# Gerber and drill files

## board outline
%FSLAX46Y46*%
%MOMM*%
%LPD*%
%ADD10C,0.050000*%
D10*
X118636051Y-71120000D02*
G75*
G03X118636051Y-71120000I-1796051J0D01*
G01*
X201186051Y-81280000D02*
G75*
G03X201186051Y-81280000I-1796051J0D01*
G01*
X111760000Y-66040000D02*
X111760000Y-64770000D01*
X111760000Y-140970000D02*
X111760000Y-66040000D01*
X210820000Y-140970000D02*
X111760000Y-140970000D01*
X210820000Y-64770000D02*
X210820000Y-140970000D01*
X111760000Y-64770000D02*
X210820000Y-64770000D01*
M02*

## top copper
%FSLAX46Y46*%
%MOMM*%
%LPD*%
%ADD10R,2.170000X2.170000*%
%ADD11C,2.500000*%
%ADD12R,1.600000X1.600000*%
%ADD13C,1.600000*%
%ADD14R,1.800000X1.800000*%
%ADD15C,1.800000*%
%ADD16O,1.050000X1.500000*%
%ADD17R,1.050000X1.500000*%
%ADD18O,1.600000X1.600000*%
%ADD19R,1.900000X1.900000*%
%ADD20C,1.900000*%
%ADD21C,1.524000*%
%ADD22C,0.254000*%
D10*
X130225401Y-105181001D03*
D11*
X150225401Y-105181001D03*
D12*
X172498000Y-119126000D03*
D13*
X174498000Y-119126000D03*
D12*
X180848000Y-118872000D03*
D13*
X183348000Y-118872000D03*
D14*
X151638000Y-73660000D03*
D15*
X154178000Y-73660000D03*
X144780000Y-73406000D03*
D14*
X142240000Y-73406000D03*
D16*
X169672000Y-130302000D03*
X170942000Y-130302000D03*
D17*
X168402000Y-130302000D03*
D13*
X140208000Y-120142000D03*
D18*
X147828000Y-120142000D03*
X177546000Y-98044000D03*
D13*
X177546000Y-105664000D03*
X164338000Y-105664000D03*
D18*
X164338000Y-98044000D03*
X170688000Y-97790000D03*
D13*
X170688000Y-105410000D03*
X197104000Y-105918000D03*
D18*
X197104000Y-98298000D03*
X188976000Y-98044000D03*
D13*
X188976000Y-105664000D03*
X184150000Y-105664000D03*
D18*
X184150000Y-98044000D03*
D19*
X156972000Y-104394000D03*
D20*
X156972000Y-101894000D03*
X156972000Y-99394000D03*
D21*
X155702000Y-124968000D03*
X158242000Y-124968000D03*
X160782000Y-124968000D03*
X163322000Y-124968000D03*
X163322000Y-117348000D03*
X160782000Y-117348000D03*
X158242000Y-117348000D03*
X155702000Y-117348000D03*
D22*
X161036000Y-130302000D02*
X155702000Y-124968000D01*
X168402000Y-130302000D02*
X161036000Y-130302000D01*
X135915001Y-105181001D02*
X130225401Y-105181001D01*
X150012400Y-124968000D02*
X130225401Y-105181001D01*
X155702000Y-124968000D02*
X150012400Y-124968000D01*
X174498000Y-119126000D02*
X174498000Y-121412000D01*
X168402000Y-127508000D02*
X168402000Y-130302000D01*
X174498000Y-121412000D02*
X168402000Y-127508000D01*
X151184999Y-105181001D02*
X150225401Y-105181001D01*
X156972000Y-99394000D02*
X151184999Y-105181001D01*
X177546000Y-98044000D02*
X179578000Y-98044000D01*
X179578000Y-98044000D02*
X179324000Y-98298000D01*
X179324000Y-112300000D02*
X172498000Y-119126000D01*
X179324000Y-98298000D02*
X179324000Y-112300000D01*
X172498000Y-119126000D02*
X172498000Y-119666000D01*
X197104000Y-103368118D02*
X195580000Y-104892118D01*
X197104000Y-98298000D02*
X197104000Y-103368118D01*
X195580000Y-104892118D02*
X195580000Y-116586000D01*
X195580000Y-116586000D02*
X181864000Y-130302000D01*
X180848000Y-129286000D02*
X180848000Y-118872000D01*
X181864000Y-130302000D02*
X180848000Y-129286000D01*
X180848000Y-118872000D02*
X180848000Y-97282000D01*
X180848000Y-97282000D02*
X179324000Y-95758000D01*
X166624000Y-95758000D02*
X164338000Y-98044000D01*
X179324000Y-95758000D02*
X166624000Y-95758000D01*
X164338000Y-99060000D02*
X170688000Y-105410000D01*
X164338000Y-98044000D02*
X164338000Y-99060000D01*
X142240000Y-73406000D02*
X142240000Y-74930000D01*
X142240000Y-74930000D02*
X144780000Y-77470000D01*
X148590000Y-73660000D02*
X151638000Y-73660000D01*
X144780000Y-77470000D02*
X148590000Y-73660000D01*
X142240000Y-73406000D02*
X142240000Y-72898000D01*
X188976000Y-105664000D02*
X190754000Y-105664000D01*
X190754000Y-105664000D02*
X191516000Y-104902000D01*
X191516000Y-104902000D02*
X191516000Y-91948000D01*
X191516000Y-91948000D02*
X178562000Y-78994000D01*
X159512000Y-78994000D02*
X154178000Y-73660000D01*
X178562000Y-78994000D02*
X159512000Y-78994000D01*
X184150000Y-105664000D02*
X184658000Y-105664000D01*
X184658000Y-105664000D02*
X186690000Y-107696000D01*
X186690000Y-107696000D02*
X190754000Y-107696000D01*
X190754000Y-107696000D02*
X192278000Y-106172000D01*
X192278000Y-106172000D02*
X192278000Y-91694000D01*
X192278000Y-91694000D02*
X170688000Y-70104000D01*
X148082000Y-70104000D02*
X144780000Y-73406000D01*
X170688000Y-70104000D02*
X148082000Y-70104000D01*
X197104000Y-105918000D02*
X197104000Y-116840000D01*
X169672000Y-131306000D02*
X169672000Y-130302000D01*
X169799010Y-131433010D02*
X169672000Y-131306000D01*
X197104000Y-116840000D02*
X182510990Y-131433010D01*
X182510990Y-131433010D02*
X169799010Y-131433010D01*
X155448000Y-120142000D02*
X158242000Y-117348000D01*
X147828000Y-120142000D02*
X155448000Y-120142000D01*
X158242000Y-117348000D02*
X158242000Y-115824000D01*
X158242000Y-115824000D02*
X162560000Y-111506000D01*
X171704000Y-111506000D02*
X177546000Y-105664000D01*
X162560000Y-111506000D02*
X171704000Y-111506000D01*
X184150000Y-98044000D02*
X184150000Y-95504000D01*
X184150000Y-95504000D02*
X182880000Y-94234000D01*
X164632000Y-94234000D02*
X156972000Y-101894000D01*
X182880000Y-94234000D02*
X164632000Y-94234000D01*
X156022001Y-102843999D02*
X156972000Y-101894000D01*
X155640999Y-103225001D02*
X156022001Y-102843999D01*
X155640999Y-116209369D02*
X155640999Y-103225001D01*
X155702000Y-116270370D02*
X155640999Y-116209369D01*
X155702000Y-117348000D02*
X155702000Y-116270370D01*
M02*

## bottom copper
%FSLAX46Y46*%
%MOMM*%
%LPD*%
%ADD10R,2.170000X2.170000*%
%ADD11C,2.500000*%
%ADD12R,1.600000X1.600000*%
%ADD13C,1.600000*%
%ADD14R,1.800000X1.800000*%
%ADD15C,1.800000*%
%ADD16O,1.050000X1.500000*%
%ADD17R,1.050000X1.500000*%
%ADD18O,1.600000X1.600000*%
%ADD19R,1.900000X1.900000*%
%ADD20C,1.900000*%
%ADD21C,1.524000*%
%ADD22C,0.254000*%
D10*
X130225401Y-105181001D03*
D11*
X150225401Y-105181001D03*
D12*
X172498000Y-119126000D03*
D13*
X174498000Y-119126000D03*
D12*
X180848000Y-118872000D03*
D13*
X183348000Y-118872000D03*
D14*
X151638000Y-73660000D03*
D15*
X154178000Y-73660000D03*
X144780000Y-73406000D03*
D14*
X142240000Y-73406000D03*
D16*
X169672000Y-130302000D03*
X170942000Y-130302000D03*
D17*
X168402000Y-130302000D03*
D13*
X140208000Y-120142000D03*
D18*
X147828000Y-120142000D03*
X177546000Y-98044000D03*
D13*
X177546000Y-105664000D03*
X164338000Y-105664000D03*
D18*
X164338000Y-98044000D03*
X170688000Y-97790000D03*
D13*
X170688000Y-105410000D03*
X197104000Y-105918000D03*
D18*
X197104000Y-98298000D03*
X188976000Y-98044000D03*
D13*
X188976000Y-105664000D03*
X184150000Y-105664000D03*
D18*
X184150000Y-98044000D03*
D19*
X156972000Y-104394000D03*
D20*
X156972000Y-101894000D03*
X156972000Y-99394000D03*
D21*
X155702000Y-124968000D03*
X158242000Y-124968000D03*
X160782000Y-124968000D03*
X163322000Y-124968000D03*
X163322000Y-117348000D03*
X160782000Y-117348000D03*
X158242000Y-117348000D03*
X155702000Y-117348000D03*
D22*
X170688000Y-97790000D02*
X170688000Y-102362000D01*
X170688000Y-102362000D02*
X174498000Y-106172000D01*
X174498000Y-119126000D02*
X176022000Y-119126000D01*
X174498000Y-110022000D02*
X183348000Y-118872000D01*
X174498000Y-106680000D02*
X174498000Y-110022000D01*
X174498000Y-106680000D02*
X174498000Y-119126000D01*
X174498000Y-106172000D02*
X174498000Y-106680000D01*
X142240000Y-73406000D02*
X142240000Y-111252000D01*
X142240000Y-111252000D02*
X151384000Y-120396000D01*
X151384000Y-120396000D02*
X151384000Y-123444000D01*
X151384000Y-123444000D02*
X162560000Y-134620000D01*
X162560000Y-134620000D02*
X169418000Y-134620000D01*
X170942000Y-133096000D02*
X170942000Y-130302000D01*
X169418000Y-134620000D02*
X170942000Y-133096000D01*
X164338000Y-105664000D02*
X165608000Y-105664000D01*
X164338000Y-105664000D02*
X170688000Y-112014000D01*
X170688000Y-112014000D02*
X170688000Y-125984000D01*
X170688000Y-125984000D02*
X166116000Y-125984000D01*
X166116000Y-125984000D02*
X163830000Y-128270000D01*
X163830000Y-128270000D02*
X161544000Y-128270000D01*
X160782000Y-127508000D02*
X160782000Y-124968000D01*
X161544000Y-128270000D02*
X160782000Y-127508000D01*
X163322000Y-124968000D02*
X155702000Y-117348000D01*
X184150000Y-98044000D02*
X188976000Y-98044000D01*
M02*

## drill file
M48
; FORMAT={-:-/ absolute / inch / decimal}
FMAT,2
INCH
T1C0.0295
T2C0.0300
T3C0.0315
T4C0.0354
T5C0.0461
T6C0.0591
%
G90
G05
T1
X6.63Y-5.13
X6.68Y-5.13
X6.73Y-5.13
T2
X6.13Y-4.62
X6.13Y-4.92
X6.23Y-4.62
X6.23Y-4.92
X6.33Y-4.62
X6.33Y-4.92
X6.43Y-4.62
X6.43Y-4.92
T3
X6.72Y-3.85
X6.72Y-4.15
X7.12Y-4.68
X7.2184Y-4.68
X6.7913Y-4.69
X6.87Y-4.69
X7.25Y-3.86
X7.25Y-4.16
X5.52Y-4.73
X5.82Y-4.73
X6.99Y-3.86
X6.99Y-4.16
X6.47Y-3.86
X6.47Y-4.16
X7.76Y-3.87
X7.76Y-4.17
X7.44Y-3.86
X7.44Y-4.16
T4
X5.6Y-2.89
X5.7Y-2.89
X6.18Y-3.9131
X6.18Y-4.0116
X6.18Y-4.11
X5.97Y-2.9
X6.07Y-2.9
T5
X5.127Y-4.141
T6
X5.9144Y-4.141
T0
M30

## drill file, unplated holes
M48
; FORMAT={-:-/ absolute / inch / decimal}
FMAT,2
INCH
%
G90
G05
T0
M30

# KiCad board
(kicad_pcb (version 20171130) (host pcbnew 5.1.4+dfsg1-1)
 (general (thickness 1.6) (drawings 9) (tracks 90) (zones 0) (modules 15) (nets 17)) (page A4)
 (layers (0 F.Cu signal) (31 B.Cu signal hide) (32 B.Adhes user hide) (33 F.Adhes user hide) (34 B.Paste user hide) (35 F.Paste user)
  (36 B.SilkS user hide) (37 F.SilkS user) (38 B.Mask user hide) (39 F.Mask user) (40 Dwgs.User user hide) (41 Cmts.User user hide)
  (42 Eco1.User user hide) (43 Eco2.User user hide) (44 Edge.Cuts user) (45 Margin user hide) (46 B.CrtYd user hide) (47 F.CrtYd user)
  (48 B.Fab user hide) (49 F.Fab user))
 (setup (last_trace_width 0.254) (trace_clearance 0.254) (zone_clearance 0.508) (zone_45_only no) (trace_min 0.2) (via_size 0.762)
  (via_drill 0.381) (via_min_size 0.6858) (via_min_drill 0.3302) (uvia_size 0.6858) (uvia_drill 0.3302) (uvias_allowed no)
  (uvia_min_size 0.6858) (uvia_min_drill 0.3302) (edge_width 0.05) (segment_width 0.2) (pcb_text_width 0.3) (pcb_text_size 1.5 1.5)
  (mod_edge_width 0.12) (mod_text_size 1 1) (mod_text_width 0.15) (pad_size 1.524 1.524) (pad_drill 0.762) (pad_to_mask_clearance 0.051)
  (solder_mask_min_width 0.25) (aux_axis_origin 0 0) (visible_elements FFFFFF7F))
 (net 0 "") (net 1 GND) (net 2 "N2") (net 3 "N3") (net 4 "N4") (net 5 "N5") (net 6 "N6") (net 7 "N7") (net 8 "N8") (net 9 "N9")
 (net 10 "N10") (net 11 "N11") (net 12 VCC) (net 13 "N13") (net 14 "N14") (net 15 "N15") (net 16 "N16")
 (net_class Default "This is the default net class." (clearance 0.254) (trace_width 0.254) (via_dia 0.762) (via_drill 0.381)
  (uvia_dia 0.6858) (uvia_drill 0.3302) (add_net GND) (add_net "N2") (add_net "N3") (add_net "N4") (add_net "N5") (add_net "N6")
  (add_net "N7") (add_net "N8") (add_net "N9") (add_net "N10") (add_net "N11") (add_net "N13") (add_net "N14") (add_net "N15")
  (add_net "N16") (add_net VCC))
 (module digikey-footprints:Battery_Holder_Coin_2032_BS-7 (layer F.Cu) (at 130.225401 105.181001)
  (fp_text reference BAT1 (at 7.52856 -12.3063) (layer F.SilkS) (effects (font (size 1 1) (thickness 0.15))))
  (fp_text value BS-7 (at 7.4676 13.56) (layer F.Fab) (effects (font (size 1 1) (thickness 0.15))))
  (pad Neg thru_hole rect (at 0 0) (size 2.17 2.17) (drill 1.17) (layers *.Cu *.Mask) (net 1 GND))
  (pad Pos thru_hole circle (at 20 0) (size 2.5 2.5) (drill 1.5) (layers *.Cu *.Mask) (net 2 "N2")))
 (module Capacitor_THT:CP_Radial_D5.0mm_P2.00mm (layer F.Cu) (at 172.498 119.126)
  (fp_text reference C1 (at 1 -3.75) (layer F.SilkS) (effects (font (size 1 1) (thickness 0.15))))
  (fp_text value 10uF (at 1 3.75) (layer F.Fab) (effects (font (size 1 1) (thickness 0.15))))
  (pad 1 thru_hole rect (at 0 0) (size 1.6 1.6) (drill 0.8) (layers *.Cu *.Mask) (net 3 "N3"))
  (pad 2 thru_hole circle (at 2 0) (size 1.6 1.6) (drill 0.8) (layers *.Cu *.Mask) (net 1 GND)))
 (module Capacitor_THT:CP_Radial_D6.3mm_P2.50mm (layer F.Cu) (at 180.848 118.872)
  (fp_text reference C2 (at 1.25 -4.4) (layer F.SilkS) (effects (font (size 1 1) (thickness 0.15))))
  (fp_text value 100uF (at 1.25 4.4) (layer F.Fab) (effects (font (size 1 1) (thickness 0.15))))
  (pad 1 thru_hole rect (at 0 0) (size 1.6 1.6) (drill 0.8) (layers *.Cu *.Mask) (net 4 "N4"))
  (pad 2 thru_hole circle (at 2.5 0) (size 1.6 1.6) (drill 0.8) (layers *.Cu *.Mask) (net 1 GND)))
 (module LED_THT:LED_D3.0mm (layer F.Cu) (at 151.638 73.66)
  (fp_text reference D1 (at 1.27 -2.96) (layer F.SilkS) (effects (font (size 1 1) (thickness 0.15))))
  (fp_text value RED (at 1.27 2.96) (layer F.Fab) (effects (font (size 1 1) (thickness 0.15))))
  (pad 1 thru_hole rect (at 0 0) (size 1.8 1.8) (drill 0.9) (layers *.Cu *.Mask) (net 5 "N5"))
  (pad 2 thru_hole circle (at 2.54 0) (size 1.8 1.8) (drill 0.9) (layers *.Cu *.Mask) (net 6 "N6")))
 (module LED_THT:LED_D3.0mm (layer F.Cu) (at 142.24 73.406)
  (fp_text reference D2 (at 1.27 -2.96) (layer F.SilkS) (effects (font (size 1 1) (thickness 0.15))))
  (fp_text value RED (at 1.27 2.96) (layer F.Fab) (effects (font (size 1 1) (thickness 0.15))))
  (pad 2 thru_hole circle (at 2.54 0) (size 1.8 1.8) (drill 0.9) (layers *.Cu *.Mask) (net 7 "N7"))
  (pad 1 thru_hole rect (at 0 0) (size 1.8 1.8) (drill 0.9) (layers *.Cu *.Mask) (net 5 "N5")))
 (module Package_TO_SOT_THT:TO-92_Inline (layer F.Cu) (at 168.402 130.302)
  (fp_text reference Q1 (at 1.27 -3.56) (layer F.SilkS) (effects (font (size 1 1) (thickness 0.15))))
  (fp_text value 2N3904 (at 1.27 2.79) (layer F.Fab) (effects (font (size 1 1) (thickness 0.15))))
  (pad 2 thru_hole oval (at 1.27 0) (size 1.05 1.5) (drill 0.75) (layers *.Cu *.Mask) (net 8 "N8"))
  (pad 3 thru_hole oval (at 2.54 0) (size 1.05 1.5) (drill 0.75) (layers *.Cu *.Mask) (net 5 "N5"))
  (pad 1 thru_hole rect (at 0 0) (size 1.05 1.5) (drill 0.75) (layers *.Cu *.Mask) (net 1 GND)))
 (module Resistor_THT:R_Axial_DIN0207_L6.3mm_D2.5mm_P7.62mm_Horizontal (layer F.Cu) (at 140.208 120.142)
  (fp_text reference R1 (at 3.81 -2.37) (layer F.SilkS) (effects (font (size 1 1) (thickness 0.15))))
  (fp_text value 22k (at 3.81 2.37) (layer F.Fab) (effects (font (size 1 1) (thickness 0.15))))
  (pad 1 thru_hole circle (at 0 0) (size 1.6 1.6) (drill 0.8) (layers *.Cu *.Mask) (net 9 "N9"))
  (pad 2 thru_hole oval (at 7.62 0) (size 1.6 1.6) (drill 0.8) (layers *.Cu *.Mask) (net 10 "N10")))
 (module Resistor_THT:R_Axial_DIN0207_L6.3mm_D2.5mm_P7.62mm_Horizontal (layer F.Cu) (at 177.546 105.664 90)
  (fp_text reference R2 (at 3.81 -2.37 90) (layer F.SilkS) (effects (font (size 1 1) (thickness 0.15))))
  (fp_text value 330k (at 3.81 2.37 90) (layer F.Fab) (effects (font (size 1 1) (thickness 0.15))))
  (pad 2 thru_hole oval (at 7.62 0 90) (size 1.6 1.6) (drill 0.8) (layers *.Cu *.Mask) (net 3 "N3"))
  (pad 1 thru_hole circle (at 0 0 90) (size 1.6 1.6) (drill 0.8) (layers *.Cu *.Mask) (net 10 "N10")))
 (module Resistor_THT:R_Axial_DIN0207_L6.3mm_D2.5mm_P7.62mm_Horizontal (layer F.Cu) (at 164.338 105.664 90)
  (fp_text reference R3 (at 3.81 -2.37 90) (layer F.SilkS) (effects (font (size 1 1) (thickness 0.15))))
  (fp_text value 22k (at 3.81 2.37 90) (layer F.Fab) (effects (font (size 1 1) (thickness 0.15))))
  (pad 1 thru_hole circle (at 0 0 90) (size 1.6 1.6) (drill 0.8) (layers *.Cu *.Mask) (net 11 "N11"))
  (pad 2 thru_hole oval (at 7.62 0 90) (size 1.6 1.6) (drill 0.8) (layers *.Cu *.Mask) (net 4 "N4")))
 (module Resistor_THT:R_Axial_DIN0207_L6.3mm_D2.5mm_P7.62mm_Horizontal (layer F.Cu) (at 170.688 105.41 90)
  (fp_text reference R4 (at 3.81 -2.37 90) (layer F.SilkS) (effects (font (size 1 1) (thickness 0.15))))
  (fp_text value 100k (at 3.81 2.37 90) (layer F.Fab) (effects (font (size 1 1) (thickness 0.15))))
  (pad 2 thru_hole oval (at 7.62 0 90) (size 1.6 1.6) (drill 0.8) (layers *.Cu *.Mask) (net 1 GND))
  (pad 1 thru_hole circle (at 0 0 90) (size 1.6 1.6) (drill 0.8) (layers *.Cu *.Mask) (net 4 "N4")))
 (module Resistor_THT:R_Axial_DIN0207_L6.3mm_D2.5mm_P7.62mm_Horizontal (layer F.Cu) (at 197.104 105.918 90)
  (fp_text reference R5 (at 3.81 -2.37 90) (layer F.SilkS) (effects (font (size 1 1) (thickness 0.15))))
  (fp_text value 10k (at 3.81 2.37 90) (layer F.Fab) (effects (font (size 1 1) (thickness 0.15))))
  (pad 1 thru_hole circle (at 0 0 90) (size 1.6 1.6) (drill 0.8) (layers *.Cu *.Mask) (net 8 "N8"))
  (pad 2 thru_hole oval (at 7.62 0 90) (size 1.6 1.6) (drill 0.8) (layers *.Cu *.Mask) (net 4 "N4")))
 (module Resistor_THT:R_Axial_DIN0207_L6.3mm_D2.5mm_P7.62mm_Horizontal (layer F.Cu) (at 188.976 105.664 90)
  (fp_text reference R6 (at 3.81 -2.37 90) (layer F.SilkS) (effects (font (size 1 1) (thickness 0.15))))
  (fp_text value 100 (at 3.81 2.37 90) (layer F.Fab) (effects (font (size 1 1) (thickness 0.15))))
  (pad 2 thru_hole oval (at 7.62 0 90) (size 1.6 1.6) (drill 0.8) (layers *.Cu *.Mask) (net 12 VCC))
  (pad 1 thru_hole circle (at 0 0 90) (size 1.6 1.6) (drill 0.8) (layers *.Cu *.Mask) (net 6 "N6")))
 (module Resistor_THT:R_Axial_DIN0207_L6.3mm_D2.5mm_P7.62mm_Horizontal (layer F.Cu) (at 184.15 105.664 90)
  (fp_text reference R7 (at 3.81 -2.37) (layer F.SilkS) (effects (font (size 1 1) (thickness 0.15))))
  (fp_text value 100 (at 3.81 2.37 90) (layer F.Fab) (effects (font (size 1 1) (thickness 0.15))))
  (pad 1 thru_hole circle (at 0 0 90) (size 1.6 1.6) (drill 0.8) (layers *.Cu *.Mask) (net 7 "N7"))
  (pad 2 thru_hole oval (at 7.62 0 90) (size 1.6 1.6) (drill 0.8) (layers *.Cu *.Mask) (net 12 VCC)))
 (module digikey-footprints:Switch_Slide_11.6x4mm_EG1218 (layer F.Cu) (at 156.972 104.394 90)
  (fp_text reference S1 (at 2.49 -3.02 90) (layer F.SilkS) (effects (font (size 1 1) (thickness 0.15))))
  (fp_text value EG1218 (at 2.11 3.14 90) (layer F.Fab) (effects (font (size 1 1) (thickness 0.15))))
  (pad 1 thru_hole rect (at 0 0 90) (size 1.9 1.9) (drill 0.9) (layers *.Cu *.Mask) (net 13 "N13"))
  (pad 2 thru_hole circle (at 2.5 0 90) (size 1.9 1.9) (drill 0.9) (layers *.Cu *.Mask) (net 12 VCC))
  (pad 3 thru_hole circle (at 5 0 90) (size 1.9 1.9) (drill 0.9) (layers *.Cu *.Mask) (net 2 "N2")))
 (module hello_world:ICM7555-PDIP (layer F.Cu) (at 159.512 121.158)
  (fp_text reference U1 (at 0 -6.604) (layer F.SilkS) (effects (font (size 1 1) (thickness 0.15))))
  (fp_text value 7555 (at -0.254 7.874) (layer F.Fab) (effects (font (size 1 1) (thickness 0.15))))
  (pad 1 thru_hole circle (at -3.81 3.81) (size 1.524 1.524) (drill 0.762) (layers *.Cu *.Mask) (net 1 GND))
  (pad 2 thru_hole circle (at -1.27 3.81) (size 1.524 1.524) (drill 0.762) (layers *.Cu *.Mask) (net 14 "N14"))
  (pad 3 thru_hole circle (at 1.27 3.81) (size 1.524 1.524) (drill 0.762) (layers *.Cu *.Mask) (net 11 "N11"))
  (pad 4 thru_hole circle (at 3.81 3.81) (size 1.524 1.524) (drill 0.762) (layers *.Cu *.Mask) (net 12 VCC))
  (pad 5 thru_hole circle (at 3.81 -3.81) (size 1.524 1.524) (drill 0.762) (layers *.Cu *.Mask) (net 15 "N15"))
  (pad 6 thru_hole circle (at 1.27 -3.81) (size 1.524 1.524) (drill 0.762) (layers *.Cu *.Mask) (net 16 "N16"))
  (pad 7 thru_hole circle (at -1.27 -3.81) (size 1.524 1.524) (drill 0.762) (layers *.Cu *.Mask) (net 10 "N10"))
  (pad 8 thru_hole circle (at -3.81 -3.81) (size 1.524 1.524) (drill 0.762) (layers *.Cu *.Mask) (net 12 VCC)))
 (gr_circle (center 116.84 71.12) (end 118.11 72.39) (layer Edge.Cuts) (width 0.05))
 (gr_circle (center 199.39 81.28) (end 200.66 82.55) (layer Edge.Cuts) (width 0.05))
 (gr_line (start 111.76 66.04) (end 111.76 64.77) (layer Edge.Cuts) (width 0.05))
 (gr_line (start 111.76 140.97) (end 111.76 66.04) (layer Edge.Cuts) (width 0.05))
 (gr_line (start 210.82 140.97) (end 111.76 140.97) (layer Edge.Cuts) (width 0.05))
 (gr_line (start 210.82 64.77) (end 210.82 140.97) (layer Edge.Cuts) (width 0.05))
 (gr_line (start 111.76 64.77) (end 210.82 64.77) (layer Edge.Cuts) (width 0.05))
 (segment (start 161.036 130.302) (end 155.702 124.968) (width 0.254) (layer F.Cu) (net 1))
 (segment (start 168.402 130.302) (end 161.036 130.302) (width 0.254) (layer F.Cu) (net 1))
 (segment (start 135.915001 105.181001) (end 130.225401 105.181001) (width 0.254) (layer F.Cu) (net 1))
 (segment (start 150.0124 124.968) (end 130.225401 105.181001) (width 0.254) (layer F.Cu) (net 1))
 (segment (start 155.702 124.968) (end 150.0124 124.968) (width 0.254) (layer F.Cu) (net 1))
 (segment (start 174.498 119.126) (end 174.498 121.412) (width 0.254) (layer F.Cu) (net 1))
 (segment (start 168.402 127.508) (end 168.402 130.302) (width 0.254) (layer F.Cu) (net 1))
 (segment (start 174.498 121.412) (end 168.402 127.508) (width 0.254) (layer F.Cu) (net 1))
 (segment (start 170.688 97.79) (end 170.688 102.362) (width 0.254) (layer B.Cu) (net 1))
 (segment (start 170.688 102.362) (end 174.498 106.172) (width 0.254) (layer B.Cu) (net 1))
 (segment (start 174.498 119.126) (end 176.022 119.126) (width 0.254) (layer B.Cu) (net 1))
 (segment (start 174.498 110.022) (end 183.348 118.872) (width 0.254) (layer B.Cu) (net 1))
 (segment (start 174.498 106.68) (end 174.498 110.022) (width 0.254) (layer B.Cu) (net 1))
 (segment (start 174.498 106.68) (end 174.498 119.126) (width 0.254) (layer B.Cu) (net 1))
 (segment (start 174.498 106.172) (end 174.498 106.68) (width 0.254) (layer B.Cu) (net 1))
 (segment (start 151.184999 105.181001) (end 150.225401 105.181001) (width 0.254) (layer F.Cu) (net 2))
 (segment (start 156.972 99.394) (end 151.184999 105.181001) (width 0.254) (layer F.Cu) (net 2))
 (segment (start 177.546 98.044) (end 179.578 98.044) (width 0.254) (layer F.Cu) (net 3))
 (segment (start 179.578 98.044) (end 179.324 98.298) (width 0.254) (layer F.Cu) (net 3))
 (segment (start 179.324 112.3) (end 172.498 119.126) (width 0.254) (layer F.Cu) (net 3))
 (segment (start 179.324 98.298) (end 179.324 112.3) (width 0.254) (layer F.Cu) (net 3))
 (segment (start 172.498 119.126) (end 172.498 119.666) (width 0.254) (layer F.Cu) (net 3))
 (segment (start 197.104 103.368118) (end 195.58 104.892118) (width 0.254) (layer F.Cu) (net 4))
 (segment (start 197.104 98.298) (end 197.104 103.368118) (width 0.254) (layer F.Cu) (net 4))
 (segment (start 195.58 104.892118) (end 195.58 116.586) (width 0.254) (layer F.Cu) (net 4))
 (segment (start 195.58 116.586) (end 181.864 130.302) (width 0.254) (layer F.Cu) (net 4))
 (segment (start 180.848 129.286) (end 180.848 118.872) (width 0.254) (layer F.Cu) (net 4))
 (segment (start 181.864 130.302) (end 180.848 129.286) (width 0.254) (layer F.Cu) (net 4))
 (segment (start 180.848 118.872) (end 180.848 97.282) (width 0.254) (layer F.Cu) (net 4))
 (segment (start 180.848 97.282) (end 179.324 95.758) (width 0.254) (layer F.Cu) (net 4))
 (segment (start 166.624 95.758) (end 164.338 98.044) (width 0.254) (layer F.Cu) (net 4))
 (segment (start 179.324 95.758) (end 166.624 95.758) (width 0.254) (layer F.Cu) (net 4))
 (segment (start 164.338 99.06) (end 170.688 105.41) (width 0.254) (layer F.Cu) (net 4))
 (segment (start 164.338 98.044) (end 164.338 99.06) (width 0.254) (layer F.Cu) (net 4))
 (segment (start 142.24 73.406) (end 142.24 74.93) (width 0.254) (layer F.Cu) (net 5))
 (segment (start 142.24 74.93) (end 144.78 77.47) (width 0.254) (layer F.Cu) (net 5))
 (segment (start 148.59 73.66) (end 151.638 73.66) (width 0.254) (layer F.Cu) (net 5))
 (segment (start 144.78 77.47) (end 148.59 73.66) (width 0.254) (layer F.Cu) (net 5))
 (segment (start 142.24 73.406) (end 142.24 72.898) (width 0.254) (layer F.Cu) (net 5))
 (segment (start 142.24 73.406) (end 142.24 111.252) (width 0.254) (layer B.Cu) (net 5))
 (segment (start 142.24 111.252) (end 151.384 120.396) (width 0.254) (layer B.Cu) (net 5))
 (segment (start 151.384 120.396) (end 151.384 123.444) (width 0.254) (layer B.Cu) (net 5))
 (segment (start 151.384 123.444) (end 162.56 134.62) (width 0.254) (layer B.Cu) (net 5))
 (segment (start 162.56 134.62) (end 169.418 134.62) (width 0.254) (layer B.Cu) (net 5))
 (segment (start 170.942 133.096) (end 170.942 130.302) (width 0.254) (layer B.Cu) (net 5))
 (segment (start 169.418 134.62) (end 170.942 133.096) (width 0.254) (layer B.Cu) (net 5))
 (segment (start 188.976 105.664) (end 190.754 105.664) (width 0.254) (layer F.Cu) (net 6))
 (segment (start 190.754 105.664) (end 191.516 104.902) (width 0.254) (layer F.Cu) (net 6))
 (segment (start 191.516 104.902) (end 191.516 91.948) (width 0.254) (layer F.Cu) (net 6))
 (segment (start 191.516 91.948) (end 178.562 78.994) (width 0.254) (layer F.Cu) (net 6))
 (segment (start 159.512 78.994) (end 154.178 73.66) (width 0.254) (layer F.Cu) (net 6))
 (segment (start 178.562 78.994) (end 159.512 78.994) (width 0.254) (layer F.Cu) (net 6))
 (segment (start 184.15 105.664) (end 184.658 105.664) (width 0.254) (layer F.Cu) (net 7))
 (segment (start 184.658 105.664) (end 186.69 107.696) (width 0.254) (layer F.Cu) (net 7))
 (segment (start 186.69 107.696) (end 190.754 107.696) (width 0.254) (layer F.Cu) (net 7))
 (segment (start 190.754 107.696) (end 192.278 106.172) (width 0.254) (layer F.Cu) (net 7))
 (segment (start 192.278 106.172) (end 192.278 91.694) (width 0.254) (layer F.Cu) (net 7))
 (segment (start 192.278 91.694) (end 170.688 70.104) (width 0.254) (layer F.Cu) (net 7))
 (segment (start 148.082 70.104) (end 144.78 73.406) (width 0.254) (layer F.Cu) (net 7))
 (segment (start 170.688 70.104) (end 148.082 70.104) (width 0.254) (layer F.Cu) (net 7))
 (segment (start 197.104 105.918) (end 197.104 116.84) (width 0.254) (layer F.Cu) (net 8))
 (segment (start 169.672 131.306) (end 169.672 130.302) (width 0.254) (layer F.Cu) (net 8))
 (segment (start 169.79901 131.43301) (end 169.672 131.306) (width 0.254) (layer F.Cu) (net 8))
 (segment (start 197.104 116.84) (end 182.51099 131.43301) (width 0.254) (layer F.Cu) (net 8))
 (segment (start 182.51099 131.43301) (end 169.79901 131.43301) (width 0.254) (layer F.Cu) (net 8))
 (segment (start 155.448 120.142) (end 158.242 117.348) (width 0.254) (layer F.Cu) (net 10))
 (segment (start 147.828 120.142) (end 155.448 120.142) (width 0.254) (layer F.Cu) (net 10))
 (segment (start 158.242 117.348) (end 158.242 115.824) (width 0.254) (layer F.Cu) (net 10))
 (segment (start 158.242 115.824) (end 162.56 111.506) (width 0.254) (layer F.Cu) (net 10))
 (segment (start 171.704 111.506) (end 177.546 105.664) (width 0.254) (layer F.Cu) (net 10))
 (segment (start 162.56 111.506) (end 171.704 111.506) (width 0.254) (layer F.Cu) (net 10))
 (segment (start 164.338 105.664) (end 165.608 105.664) (width 0.254) (layer B.Cu) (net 11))
 (segment (start 164.338 105.664) (end 170.688 112.014) (width 0.254) (layer B.Cu) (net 11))
 (segment (start 170.688 112.014) (end 170.688 125.984) (width 0.254) (layer B.Cu) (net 11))
 (segment (start 170.688 125.984) (end 166.116 125.984) (width 0.254) (layer B.Cu) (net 11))
 (segment (start 166.116 125.984) (end 163.83 128.27) (width 0.254) (layer B.Cu) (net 11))
 (segment (start 163.83 128.27) (end 161.544 128.27) (width 0.254) (layer B.Cu) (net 11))
 (segment (start 160.782 127.508) (end 160.782 124.968) (width 0.254) (layer B.Cu) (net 11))
 (segment (start 161.544 128.27) (end 160.782 127.508) (width 0.254) (layer B.Cu) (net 11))
 (segment (start 184.15 98.044) (end 184.15 95.504) (width 0.254) (layer F.Cu) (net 12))
 (segment (start 184.15 95.504) (end 182.88 94.234) (width 0.254) (layer F.Cu) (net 12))
 (segment (start 164.632 94.234) (end 156.972 101.894) (width 0.254) (layer F.Cu) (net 12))
 (segment (start 182.88 94.234) (end 164.632 94.234) (width 0.254) (layer F.Cu) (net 12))
 (segment (start 156.022001 102.843999) (end 156.972 101.894) (width 0.254) (layer F.Cu) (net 12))
 (segment (start 155.640999 103.225001) (end 156.022001 102.843999) (width 0.254) (layer F.Cu) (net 12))
 (segment (start 155.640999 116.209369) (end 155.640999 103.225001) (width 0.254) (layer F.Cu) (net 12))
 (segment (start 155.702 116.27037) (end 155.640999 116.209369) (width 0.254) (layer F.Cu) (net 12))
 (segment (start 155.702 117.348) (end 155.702 116.27037) (width 0.254) (layer F.Cu) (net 12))
 (segment (start 163.322 124.968) (end 155.702 117.348) (width 0.254) (layer B.Cu) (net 12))
 (segment (start 184.15 98.044) (end 188.976 98.044) (width 0.254) (layer B.Cu) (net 12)))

